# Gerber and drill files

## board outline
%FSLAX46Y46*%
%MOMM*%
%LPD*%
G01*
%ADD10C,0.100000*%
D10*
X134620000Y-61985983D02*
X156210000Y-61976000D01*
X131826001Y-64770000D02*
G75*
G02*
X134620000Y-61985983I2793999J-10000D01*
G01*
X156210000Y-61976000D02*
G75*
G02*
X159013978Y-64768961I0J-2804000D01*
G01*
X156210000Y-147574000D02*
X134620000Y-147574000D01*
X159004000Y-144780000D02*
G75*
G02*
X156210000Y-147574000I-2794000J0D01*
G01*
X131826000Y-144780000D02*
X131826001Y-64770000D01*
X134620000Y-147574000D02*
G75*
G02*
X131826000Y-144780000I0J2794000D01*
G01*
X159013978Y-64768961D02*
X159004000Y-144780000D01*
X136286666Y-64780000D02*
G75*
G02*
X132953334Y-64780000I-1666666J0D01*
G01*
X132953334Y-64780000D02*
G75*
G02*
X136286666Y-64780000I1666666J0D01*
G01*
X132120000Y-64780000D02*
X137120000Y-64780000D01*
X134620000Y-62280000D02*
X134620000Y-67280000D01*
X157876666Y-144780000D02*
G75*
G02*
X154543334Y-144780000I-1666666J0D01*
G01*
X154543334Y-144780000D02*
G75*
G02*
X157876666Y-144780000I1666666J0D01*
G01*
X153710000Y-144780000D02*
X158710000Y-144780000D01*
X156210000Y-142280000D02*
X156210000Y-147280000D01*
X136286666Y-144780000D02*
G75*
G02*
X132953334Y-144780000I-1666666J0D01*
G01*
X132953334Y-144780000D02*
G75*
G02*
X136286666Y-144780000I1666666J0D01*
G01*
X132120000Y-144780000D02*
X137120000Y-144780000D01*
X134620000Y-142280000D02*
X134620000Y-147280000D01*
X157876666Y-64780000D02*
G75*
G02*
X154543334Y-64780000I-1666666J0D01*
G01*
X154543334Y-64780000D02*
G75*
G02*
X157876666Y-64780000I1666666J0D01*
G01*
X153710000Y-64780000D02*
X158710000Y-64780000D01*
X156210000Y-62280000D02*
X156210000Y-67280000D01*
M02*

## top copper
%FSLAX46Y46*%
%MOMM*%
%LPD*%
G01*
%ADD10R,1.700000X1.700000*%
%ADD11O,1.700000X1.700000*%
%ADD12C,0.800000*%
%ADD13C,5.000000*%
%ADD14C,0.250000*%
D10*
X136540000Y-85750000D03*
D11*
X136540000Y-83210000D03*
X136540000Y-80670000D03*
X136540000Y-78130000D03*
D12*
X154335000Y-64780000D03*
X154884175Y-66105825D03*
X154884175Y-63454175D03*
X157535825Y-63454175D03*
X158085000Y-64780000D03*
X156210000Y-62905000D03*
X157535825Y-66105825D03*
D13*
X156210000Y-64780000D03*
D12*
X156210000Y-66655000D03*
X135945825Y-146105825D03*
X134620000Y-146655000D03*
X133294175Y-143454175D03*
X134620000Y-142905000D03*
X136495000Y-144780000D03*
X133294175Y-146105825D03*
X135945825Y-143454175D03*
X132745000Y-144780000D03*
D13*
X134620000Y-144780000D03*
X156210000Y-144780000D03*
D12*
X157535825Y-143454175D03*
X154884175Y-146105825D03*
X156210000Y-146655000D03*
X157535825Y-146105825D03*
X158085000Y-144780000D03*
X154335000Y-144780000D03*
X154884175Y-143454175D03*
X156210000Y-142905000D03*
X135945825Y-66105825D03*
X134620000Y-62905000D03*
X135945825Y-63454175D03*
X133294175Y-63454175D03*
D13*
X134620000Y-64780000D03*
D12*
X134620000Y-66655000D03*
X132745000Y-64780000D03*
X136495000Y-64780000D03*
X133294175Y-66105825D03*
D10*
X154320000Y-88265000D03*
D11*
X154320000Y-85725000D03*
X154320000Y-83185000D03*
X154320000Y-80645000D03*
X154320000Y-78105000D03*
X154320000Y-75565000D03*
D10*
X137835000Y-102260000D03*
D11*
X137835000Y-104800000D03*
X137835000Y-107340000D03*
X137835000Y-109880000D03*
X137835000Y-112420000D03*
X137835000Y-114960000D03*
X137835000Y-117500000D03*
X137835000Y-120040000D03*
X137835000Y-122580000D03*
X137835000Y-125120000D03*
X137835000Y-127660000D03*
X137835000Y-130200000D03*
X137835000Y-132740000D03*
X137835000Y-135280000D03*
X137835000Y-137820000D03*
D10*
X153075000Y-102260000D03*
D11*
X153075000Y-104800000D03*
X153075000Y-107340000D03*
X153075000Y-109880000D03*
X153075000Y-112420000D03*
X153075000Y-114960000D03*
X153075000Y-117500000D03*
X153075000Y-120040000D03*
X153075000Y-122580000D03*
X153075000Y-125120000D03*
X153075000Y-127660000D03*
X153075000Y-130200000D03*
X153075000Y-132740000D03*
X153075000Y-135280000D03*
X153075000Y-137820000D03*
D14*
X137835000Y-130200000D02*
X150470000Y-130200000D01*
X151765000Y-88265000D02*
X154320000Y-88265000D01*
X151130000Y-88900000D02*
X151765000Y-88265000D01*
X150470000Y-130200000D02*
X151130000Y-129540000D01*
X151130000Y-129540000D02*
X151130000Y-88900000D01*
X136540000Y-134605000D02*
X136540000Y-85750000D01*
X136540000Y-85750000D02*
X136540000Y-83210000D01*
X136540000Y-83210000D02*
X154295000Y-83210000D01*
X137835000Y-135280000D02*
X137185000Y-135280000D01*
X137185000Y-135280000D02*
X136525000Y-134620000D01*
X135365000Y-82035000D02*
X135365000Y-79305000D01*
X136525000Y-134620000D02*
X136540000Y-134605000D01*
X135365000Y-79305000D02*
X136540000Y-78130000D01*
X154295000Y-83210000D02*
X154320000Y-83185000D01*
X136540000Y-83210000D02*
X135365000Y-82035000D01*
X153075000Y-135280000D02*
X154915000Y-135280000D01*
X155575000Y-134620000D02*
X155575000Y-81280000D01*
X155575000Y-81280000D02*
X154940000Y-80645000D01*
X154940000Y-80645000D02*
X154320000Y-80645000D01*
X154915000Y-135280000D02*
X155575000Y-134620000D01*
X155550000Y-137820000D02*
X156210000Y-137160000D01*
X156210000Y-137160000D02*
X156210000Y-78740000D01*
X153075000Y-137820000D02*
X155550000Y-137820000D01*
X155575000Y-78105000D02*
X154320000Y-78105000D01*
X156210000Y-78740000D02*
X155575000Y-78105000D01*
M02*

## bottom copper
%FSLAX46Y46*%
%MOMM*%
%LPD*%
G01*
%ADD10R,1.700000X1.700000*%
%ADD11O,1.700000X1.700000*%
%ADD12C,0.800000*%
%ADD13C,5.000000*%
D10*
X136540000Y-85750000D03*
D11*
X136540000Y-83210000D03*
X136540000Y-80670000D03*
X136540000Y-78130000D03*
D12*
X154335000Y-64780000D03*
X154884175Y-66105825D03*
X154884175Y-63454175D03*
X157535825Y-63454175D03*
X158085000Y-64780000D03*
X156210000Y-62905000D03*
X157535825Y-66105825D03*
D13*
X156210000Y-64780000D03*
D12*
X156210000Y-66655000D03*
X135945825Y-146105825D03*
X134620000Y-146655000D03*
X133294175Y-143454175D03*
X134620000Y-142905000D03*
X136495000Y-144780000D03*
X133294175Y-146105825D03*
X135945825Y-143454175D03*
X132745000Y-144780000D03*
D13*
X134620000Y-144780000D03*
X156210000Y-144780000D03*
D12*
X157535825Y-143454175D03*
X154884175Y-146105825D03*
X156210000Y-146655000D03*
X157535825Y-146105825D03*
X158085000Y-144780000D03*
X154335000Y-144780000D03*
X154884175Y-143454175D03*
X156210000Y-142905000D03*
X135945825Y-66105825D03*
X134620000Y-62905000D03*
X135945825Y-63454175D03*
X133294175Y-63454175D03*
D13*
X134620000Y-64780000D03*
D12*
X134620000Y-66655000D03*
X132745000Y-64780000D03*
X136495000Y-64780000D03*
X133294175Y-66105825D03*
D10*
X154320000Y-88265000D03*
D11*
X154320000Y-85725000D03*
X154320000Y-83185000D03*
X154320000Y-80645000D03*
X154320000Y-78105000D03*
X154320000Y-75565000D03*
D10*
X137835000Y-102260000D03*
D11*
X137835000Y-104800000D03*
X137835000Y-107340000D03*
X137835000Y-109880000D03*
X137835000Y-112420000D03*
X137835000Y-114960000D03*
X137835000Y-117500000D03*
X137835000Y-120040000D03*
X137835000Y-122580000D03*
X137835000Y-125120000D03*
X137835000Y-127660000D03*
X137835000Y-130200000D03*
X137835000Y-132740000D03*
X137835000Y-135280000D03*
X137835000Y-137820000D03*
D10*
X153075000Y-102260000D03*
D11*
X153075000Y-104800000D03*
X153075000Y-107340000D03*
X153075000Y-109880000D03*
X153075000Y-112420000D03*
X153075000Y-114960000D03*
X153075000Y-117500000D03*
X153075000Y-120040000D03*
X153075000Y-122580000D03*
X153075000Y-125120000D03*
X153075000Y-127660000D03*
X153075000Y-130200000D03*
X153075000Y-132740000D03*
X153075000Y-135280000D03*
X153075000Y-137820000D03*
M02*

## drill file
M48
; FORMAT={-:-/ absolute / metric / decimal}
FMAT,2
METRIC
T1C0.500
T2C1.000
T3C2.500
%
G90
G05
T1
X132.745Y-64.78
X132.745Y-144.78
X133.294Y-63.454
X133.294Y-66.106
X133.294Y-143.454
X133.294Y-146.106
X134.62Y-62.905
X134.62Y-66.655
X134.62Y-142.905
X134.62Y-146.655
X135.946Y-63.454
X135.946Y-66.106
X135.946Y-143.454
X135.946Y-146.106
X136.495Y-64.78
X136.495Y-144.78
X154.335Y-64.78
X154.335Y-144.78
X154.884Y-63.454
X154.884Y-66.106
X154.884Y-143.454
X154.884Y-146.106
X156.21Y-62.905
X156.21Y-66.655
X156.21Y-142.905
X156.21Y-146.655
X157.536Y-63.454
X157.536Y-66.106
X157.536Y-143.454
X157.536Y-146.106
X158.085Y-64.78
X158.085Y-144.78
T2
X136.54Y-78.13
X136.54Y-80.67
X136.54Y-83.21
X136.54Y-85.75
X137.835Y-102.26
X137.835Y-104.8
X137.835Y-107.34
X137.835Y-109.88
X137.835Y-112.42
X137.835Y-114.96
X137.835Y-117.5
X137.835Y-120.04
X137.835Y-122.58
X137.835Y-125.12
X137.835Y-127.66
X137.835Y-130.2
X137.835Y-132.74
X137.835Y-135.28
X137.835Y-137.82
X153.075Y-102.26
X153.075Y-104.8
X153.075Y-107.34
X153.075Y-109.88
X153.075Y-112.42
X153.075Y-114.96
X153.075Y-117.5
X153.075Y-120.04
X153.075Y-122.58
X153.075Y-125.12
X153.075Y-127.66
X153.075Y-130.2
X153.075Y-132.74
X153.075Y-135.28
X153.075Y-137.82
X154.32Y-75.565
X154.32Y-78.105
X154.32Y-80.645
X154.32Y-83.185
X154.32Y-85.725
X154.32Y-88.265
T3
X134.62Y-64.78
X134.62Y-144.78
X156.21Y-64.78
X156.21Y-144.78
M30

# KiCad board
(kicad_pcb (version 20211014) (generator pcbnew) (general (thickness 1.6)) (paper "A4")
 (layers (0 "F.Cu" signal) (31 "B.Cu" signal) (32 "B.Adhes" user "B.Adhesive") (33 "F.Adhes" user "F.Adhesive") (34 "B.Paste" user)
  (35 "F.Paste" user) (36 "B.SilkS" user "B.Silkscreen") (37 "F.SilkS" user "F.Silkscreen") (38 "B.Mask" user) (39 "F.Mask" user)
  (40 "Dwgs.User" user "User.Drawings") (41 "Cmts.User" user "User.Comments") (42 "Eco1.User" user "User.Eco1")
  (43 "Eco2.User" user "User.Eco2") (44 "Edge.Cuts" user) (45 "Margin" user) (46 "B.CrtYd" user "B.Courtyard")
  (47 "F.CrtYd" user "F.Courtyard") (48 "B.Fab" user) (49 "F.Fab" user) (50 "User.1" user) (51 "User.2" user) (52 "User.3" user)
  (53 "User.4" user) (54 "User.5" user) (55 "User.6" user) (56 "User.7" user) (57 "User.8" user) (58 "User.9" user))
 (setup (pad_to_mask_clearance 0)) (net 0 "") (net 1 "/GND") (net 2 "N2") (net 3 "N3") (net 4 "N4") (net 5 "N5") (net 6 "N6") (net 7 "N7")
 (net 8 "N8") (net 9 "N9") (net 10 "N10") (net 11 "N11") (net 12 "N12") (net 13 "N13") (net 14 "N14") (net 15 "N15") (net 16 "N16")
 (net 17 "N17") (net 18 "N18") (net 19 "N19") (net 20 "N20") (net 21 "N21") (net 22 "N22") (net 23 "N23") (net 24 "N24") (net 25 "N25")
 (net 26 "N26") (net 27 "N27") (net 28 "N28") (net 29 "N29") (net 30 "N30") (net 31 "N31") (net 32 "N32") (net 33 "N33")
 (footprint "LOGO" (layer "F.Cu") (at 145.415 69.85)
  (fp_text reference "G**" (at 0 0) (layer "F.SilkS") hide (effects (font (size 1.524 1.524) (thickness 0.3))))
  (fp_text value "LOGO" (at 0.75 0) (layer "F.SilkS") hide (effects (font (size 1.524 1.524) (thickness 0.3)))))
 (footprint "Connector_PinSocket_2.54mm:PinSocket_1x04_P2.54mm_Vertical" (layer "F.Cu") (at 136.54 85.75 180)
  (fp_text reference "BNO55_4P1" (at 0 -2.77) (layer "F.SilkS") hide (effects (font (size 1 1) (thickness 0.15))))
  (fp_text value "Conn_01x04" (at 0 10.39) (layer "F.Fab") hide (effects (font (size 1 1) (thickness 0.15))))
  (pad "1" thru_hole rect (at 0 0 180) (size 1.7 1.7) (drill 1) (layers *.Cu *.Mask) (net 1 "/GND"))
  (pad "2" thru_hole oval (at 0 2.54 180) (size 1.7 1.7) (drill 1) (layers *.Cu *.Mask) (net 1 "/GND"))
  (pad "3" thru_hole oval (at 0 5.08 180) (size 1.7 1.7) (drill 1) (layers *.Cu *.Mask) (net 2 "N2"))
  (pad "4" thru_hole oval (at 0 7.62 180) (size 1.7 1.7) (drill 1) (layers *.Cu *.Mask) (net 1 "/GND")))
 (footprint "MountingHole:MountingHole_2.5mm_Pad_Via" (layer "F.Cu") (at 156.21 64.78)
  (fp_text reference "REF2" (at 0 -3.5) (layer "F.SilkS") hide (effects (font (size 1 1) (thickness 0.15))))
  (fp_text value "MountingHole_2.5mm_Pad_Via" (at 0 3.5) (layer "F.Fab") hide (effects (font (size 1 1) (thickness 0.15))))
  (pad "1" thru_hole circle (at -1.875 0) (size 0.8 0.8) (drill 0.5) (layers F&B.Cu *.Mask))
  (pad "1" thru_hole circle (at -1.325825 1.325825) (size 0.8 0.8) (drill 0.5) (layers F&B.Cu *.Mask))
  (pad "1" thru_hole circle (at -1.325825 -1.325825) (size 0.8 0.8) (drill 0.5) (layers F&B.Cu *.Mask))
  (pad "1" thru_hole circle (at 1.325825 -1.325825) (size 0.8 0.8) (drill 0.5) (layers F&B.Cu *.Mask))
  (pad "1" thru_hole circle (at 1.875 0) (size 0.8 0.8) (drill 0.5) (layers F&B.Cu *.Mask))
  (pad "1" thru_hole circle (at 0 -1.875) (size 0.8 0.8) (drill 0.5) (layers F&B.Cu *.Mask))
  (pad "1" thru_hole circle (at 1.325825 1.325825) (size 0.8 0.8) (drill 0.5) (layers F&B.Cu *.Mask))
  (pad "1" thru_hole circle (at 0 0) (size 5 5) (drill 2.5) (layers F&B.Cu *.Mask))
  (pad "1" thru_hole circle (at 0 1.875) (size 0.8 0.8) (drill 0.5) (layers F&B.Cu *.Mask)))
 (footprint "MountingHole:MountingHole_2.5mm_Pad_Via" (layer "F.Cu") (at 134.62 144.78)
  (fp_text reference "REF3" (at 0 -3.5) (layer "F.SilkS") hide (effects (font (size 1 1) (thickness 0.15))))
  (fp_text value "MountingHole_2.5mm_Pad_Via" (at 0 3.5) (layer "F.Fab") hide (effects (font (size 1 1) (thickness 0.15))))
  (pad "1" thru_hole circle (at 1.325825 1.325825) (size 0.8 0.8) (drill 0.5) (layers *.Cu *.Mask))
  (pad "1" thru_hole circle (at 0 1.875) (size 0.8 0.8) (drill 0.5) (layers *.Cu *.Mask))
  (pad "1" thru_hole circle (at -1.325825 -1.325825) (size 0.8 0.8) (drill 0.5) (layers *.Cu *.Mask))
  (pad "1" thru_hole circle (at 0 -1.875) (size 0.8 0.8) (drill 0.5) (layers *.Cu *.Mask))
  (pad "1" thru_hole circle (at 1.875 0) (size 0.8 0.8) (drill 0.5) (layers *.Cu *.Mask))
  (pad "1" thru_hole circle (at -1.325825 1.325825) (size 0.8 0.8) (drill 0.5) (layers *.Cu *.Mask))
  (pad "1" thru_hole circle (at 1.325825 -1.325825) (size 0.8 0.8) (drill 0.5) (layers *.Cu *.Mask))
  (pad "1" thru_hole circle (at -1.875 0) (size 0.8 0.8) (drill 0.5) (layers *.Cu *.Mask))
  (pad "1" thru_hole circle (at 0 0) (size 5 5) (drill 2.5) (layers *.Cu *.Mask)))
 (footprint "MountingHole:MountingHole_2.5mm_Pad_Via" (layer "F.Cu") (at 156.21 144.78)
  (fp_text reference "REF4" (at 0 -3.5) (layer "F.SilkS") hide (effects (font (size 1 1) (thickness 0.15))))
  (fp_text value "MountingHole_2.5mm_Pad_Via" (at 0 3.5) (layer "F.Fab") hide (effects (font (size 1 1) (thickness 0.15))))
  (pad "1" thru_hole circle (at 0 0) (size 5 5) (drill 2.5) (layers *.Cu *.Mask))
  (pad "1" thru_hole circle (at 1.325825 -1.325825) (size 0.8 0.8) (drill 0.5) (layers *.Cu *.Mask))
  (pad "1" thru_hole circle (at -1.325825 1.325825) (size 0.8 0.8) (drill 0.5) (layers *.Cu *.Mask))
  (pad "1" thru_hole circle (at 0 1.875) (size 0.8 0.8) (drill 0.5) (layers *.Cu *.Mask))
  (pad "1" thru_hole circle (at 1.325825 1.325825) (size 0.8 0.8) (drill 0.5) (layers *.Cu *.Mask))
  (pad "1" thru_hole circle (at 1.875 0) (size 0.8 0.8) (drill 0.5) (layers *.Cu *.Mask))
  (pad "1" thru_hole circle (at -1.875 0) (size 0.8 0.8) (drill 0.5) (layers *.Cu *.Mask))
  (pad "1" thru_hole circle (at -1.325825 -1.325825) (size 0.8 0.8) (drill 0.5) (layers *.Cu *.Mask))
  (pad "1" thru_hole circle (at 0 -1.875) (size 0.8 0.8) (drill 0.5) (layers *.Cu *.Mask)))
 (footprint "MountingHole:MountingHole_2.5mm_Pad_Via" (layer "F.Cu") (at 134.62 64.78)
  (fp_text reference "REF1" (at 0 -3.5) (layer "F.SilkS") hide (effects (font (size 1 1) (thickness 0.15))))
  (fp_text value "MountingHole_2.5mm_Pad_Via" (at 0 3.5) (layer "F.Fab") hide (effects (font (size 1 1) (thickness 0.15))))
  (pad "1" thru_hole circle (at 1.325825 1.325825) (size 0.8 0.8) (drill 0.5) (layers F&B.Cu *.Mask))
  (pad "1" thru_hole circle (at 0 -1.875) (size 0.8 0.8) (drill 0.5) (layers F&B.Cu *.Mask))
  (pad "1" thru_hole circle (at 1.325825 -1.325825) (size 0.8 0.8) (drill 0.5) (layers F&B.Cu *.Mask))
  (pad "1" thru_hole circle (at -1.325825 -1.325825) (size 0.8 0.8) (drill 0.5) (layers F&B.Cu *.Mask))
  (pad "1" thru_hole circle (at 0 0) (size 5 5) (drill 2.5) (layers F&B.Cu *.Mask))
  (pad "1" thru_hole circle (at 0 1.875) (size 0.8 0.8) (drill 0.5) (layers F&B.Cu *.Mask))
  (pad "1" thru_hole circle (at -1.875 0) (size 0.8 0.8) (drill 0.5) (layers F&B.Cu *.Mask))
  (pad "1" thru_hole circle (at 1.875 0) (size 0.8 0.8) (drill 0.5) (layers F&B.Cu *.Mask))
  (pad "1" thru_hole circle (at -1.325825 1.325825) (size 0.8 0.8) (drill 0.5) (layers F&B.Cu *.Mask)))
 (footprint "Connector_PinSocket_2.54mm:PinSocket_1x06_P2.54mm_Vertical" (layer "F.Cu") (at 154.32 88.265 180)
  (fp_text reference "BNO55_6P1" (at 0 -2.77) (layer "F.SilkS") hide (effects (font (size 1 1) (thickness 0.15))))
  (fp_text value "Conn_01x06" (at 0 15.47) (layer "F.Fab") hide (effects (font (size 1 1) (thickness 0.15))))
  (pad "1" thru_hole rect (at 0 0 180) (size 1.7 1.7) (drill 1) (layers *.Cu *.Mask) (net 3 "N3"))
  (pad "2" thru_hole oval (at 0 2.54 180) (size 1.7 1.7) (drill 1) (layers *.Cu *.Mask) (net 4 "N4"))
  (pad "3" thru_hole oval (at 0 5.08 180) (size 1.7 1.7) (drill 1) (layers *.Cu *.Mask) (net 1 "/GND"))
  (pad "4" thru_hole oval (at 0 7.62 180) (size 1.7 1.7) (drill 1) (layers *.Cu *.Mask) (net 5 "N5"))
  (pad "5" thru_hole oval (at 0 10.16 180) (size 1.7 1.7) (drill 1) (layers *.Cu *.Mask) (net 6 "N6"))
  (pad "6" thru_hole oval (at 0 12.7 180) (size 1.7 1.7) (drill 1) (layers *.Cu *.Mask) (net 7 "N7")))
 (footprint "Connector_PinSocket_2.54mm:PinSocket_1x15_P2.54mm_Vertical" (layer "B.Cu") (at 137.835 102.26 180)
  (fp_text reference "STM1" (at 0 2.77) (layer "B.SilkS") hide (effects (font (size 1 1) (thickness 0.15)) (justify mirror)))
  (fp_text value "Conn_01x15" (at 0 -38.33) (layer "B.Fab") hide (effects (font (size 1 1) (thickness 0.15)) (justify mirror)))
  (pad "1" thru_hole rect (at 0 0 180) (size 1.7 1.7) (drill 1) (layers *.Cu *.Mask) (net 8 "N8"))
  (pad "2" thru_hole oval (at 0 -2.54 180) (size 1.7 1.7) (drill 1) (layers *.Cu *.Mask) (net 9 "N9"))
  (pad "3" thru_hole oval (at 0 -5.08 180) (size 1.7 1.7) (drill 1) (layers *.Cu *.Mask) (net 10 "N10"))
  (pad "4" thru_hole oval (at 0 -7.62 180) (size 1.7 1.7) (drill 1) (layers *.Cu *.Mask) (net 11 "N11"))
  (pad "5" thru_hole oval (at 0 -10.16 180) (size 1.7 1.7) (drill 1) (layers *.Cu *.Mask) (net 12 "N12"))
  (pad "6" thru_hole oval (at 0 -12.7 180) (size 1.7 1.7) (drill 1) (layers *.Cu *.Mask) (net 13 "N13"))
  (pad "7" thru_hole oval (at 0 -15.24 180) (size 1.7 1.7) (drill 1) (layers *.Cu *.Mask) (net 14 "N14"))
  (pad "8" thru_hole oval (at 0 -17.78 180) (size 1.7 1.7) (drill 1) (layers *.Cu *.Mask) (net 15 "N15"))
  (pad "9" thru_hole oval (at 0 -20.32 180) (size 1.7 1.7) (drill 1) (layers *.Cu *.Mask) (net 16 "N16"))
  (pad "10" thru_hole oval (at 0 -22.86 180) (size 1.7 1.7) (drill 1) (layers *.Cu *.Mask) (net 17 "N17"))
  (pad "11" thru_hole oval (at 0 -25.4 180) (size 1.7 1.7) (drill 1) (layers *.Cu *.Mask) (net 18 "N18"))
  (pad "12" thru_hole oval (at 0 -27.94 180) (size 1.7 1.7) (drill 1) (layers *.Cu *.Mask) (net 3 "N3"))
  (pad "13" thru_hole oval (at 0 -30.48 180) (size 1.7 1.7) (drill 1) (layers *.Cu *.Mask) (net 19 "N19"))
  (pad "14" thru_hole oval (at 0 -33.02 180) (size 1.7 1.7) (drill 1) (layers *.Cu *.Mask) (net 1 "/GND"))
  (pad "15" thru_hole oval (at 0 -35.56 180) (size 1.7 1.7) (drill 1) (layers *.Cu *.Mask) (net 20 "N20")))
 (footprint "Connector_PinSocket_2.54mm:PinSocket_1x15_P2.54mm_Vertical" (layer "B.Cu") (at 153.075 102.26 180)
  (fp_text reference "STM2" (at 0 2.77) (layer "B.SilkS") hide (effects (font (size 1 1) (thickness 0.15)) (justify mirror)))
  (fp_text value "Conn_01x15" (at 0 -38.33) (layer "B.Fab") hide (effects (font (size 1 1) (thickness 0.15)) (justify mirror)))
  (pad "1" thru_hole rect (at 0 0 180) (size 1.7 1.7) (drill 1) (layers *.Cu *.Mask) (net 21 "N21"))
  (pad "2" thru_hole oval (at 0 -2.54 180) (size 1.7 1.7) (drill 1) (layers *.Cu *.Mask) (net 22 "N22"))
  (pad "3" thru_hole oval (at 0 -5.08 180) (size 1.7 1.7) (drill 1) (layers *.Cu *.Mask) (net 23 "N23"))
  (pad "4" thru_hole oval (at 0 -7.62 180) (size 1.7 1.7) (drill 1) (layers *.Cu *.Mask) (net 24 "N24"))
  (pad "5" thru_hole oval (at 0 -10.16 180) (size 1.7 1.7) (drill 1) (layers *.Cu *.Mask) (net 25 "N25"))
  (pad "6" thru_hole oval (at 0 -12.7 180) (size 1.7 1.7) (drill 1) (layers *.Cu *.Mask) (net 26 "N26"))
  (pad "7" thru_hole oval (at 0 -15.24 180) (size 1.7 1.7) (drill 1) (layers *.Cu *.Mask) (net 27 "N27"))
  (pad "8" thru_hole oval (at 0 -17.78 180) (size 1.7 1.7) (drill 1) (layers *.Cu *.Mask) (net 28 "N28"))
  (pad "9" thru_hole oval (at 0 -20.32 180) (size 1.7 1.7) (drill 1) (layers *.Cu *.Mask) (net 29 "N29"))
  (pad "10" thru_hole oval (at 0 -22.86 180) (size 1.7 1.7) (drill 1) (layers *.Cu *.Mask) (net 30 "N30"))
  (pad "11" thru_hole oval (at 0 -25.4 180) (size 1.7 1.7) (drill 1) (layers *.Cu *.Mask) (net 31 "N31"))
  (pad "12" thru_hole oval (at 0 -27.94 180) (size 1.7 1.7) (drill 1) (layers *.Cu *.Mask) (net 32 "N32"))
  (pad "13" thru_hole oval (at 0 -30.48 180) (size 1.7 1.7) (drill 1) (layers *.Cu *.Mask) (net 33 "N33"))
  (pad "14" thru_hole oval (at 0 -33.02 180) (size 1.7 1.7) (drill 1) (layers *.Cu *.Mask) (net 5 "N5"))
  (pad "15" thru_hole oval (at 0 -35.56 180) (size 1.7 1.7) (drill 1) (layers *.Cu *.Mask) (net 6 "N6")))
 (gr_line (start 134.62 61.985983) (end 156.21 61.976) (layer "Edge.Cuts") (width 0.1))
 (gr_arc (start 131.826001 64.77) (mid 132.64787 62.800799) (end 134.62 61.985983) (layer "Edge.Cuts") (width 0.1))
 (gr_arc (start 156.21 61.976) (mid 158.188821 62.793374) (end 159.013978 64.768961) (layer "Edge.Cuts") (width 0.1))
 (gr_line (start 156.21 147.574) (end 134.62 147.574) (layer "Edge.Cuts") (width 0.1))
 (gr_arc (start 159.004 144.78) (mid 158.185656 146.755656) (end 156.21 147.574) (layer "Edge.Cuts") (width 0.1))
 (gr_line (start 131.826 144.78) (end 131.826001 64.77) (layer "Edge.Cuts") (width 0.1))
 (gr_arc (start 134.62 147.574) (mid 132.644344 146.755656) (end 131.826 144.78) (layer "Edge.Cuts") (width 0.1))
 (gr_line (start 159.013978 64.768961) (end 159.004 144.78) (layer "Edge.Cuts") (width 0.1))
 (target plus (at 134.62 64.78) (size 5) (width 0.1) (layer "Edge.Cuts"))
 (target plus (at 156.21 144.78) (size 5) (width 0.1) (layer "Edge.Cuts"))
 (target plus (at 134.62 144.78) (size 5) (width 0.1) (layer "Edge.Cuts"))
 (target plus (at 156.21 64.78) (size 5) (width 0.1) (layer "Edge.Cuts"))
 (segment (start 137.835 130.2) (end 150.47 130.2) (width 0.25) (layer "F.Cu") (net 3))
 (segment (start 151.765 88.265) (end 154.32 88.265) (width 0.25) (layer "F.Cu") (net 3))
 (segment (start 151.13 88.9) (end 151.765 88.265) (width 0.25) (layer "F.Cu") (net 3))
 (segment (start 150.47 130.2) (end 151.13 129.54) (width 0.25) (layer "F.Cu") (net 3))
 (segment (start 151.13 129.54) (end 151.13 88.9) (width 0.25) (layer "F.Cu") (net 3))
 (segment (start 136.54 134.605) (end 136.54 85.75) (width 0.25) (layer "F.Cu") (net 1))
 (segment (start 136.54 85.75) (end 136.54 83.21) (width 0.25) (layer "F.Cu") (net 1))
 (segment (start 136.54 83.21) (end 154.295 83.21) (width 0.25) (layer "F.Cu") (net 1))
 (segment (start 137.835 135.28) (end 137.185 135.28) (width 0.25) (layer "F.Cu") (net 1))
 (segment (start 137.185 135.28) (end 136.525 134.62) (width 0.25) (layer "F.Cu") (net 1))
 (segment (start 135.365 82.035) (end 135.365 79.305) (width 0.25) (layer "F.Cu") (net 1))
 (segment (start 136.525 134.62) (end 136.54 134.605) (width 0.25) (layer "F.Cu") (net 1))
 (segment (start 135.365 79.305) (end 136.54 78.13) (width 0.25) (layer "F.Cu") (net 1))
 (segment (start 154.295 83.21) (end 154.32 83.185) (width 0.25) (layer "F.Cu") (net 1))
 (segment (start 136.54 83.21) (end 135.365 82.035) (width 0.25) (layer "F.Cu") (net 1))
 (segment (start 153.075 135.28) (end 154.915 135.28) (width 0.25) (layer "F.Cu") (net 5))
 (segment (start 155.575 134.62) (end 155.575 81.28) (width 0.25) (layer "F.Cu") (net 5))
 (segment (start 155.575 81.28) (end 154.94 80.645) (width 0.25) (layer "F.Cu") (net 5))
 (segment (start 154.94 80.645) (end 154.32 80.645) (width 0.25) (layer "F.Cu") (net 5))
 (segment (start 154.915 135.28) (end 155.575 134.62) (width 0.25) (layer "F.Cu") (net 5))
 (segment (start 155.55 137.82) (end 156.21 137.16) (width 0.25) (layer "F.Cu") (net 6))
 (segment (start 156.21 137.16) (end 156.21 78.74) (width 0.25) (layer "F.Cu") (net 6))
 (segment (start 153.075 137.82) (end 155.55 137.82) (width 0.25) (layer "F.Cu") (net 6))
 (segment (start 155.575 78.105) (end 154.32 78.105) (width 0.25) (layer "F.Cu") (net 6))
 (segment (start 156.21 78.74) (end 155.575 78.105) (width 0.25) (layer "F.Cu") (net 6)))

